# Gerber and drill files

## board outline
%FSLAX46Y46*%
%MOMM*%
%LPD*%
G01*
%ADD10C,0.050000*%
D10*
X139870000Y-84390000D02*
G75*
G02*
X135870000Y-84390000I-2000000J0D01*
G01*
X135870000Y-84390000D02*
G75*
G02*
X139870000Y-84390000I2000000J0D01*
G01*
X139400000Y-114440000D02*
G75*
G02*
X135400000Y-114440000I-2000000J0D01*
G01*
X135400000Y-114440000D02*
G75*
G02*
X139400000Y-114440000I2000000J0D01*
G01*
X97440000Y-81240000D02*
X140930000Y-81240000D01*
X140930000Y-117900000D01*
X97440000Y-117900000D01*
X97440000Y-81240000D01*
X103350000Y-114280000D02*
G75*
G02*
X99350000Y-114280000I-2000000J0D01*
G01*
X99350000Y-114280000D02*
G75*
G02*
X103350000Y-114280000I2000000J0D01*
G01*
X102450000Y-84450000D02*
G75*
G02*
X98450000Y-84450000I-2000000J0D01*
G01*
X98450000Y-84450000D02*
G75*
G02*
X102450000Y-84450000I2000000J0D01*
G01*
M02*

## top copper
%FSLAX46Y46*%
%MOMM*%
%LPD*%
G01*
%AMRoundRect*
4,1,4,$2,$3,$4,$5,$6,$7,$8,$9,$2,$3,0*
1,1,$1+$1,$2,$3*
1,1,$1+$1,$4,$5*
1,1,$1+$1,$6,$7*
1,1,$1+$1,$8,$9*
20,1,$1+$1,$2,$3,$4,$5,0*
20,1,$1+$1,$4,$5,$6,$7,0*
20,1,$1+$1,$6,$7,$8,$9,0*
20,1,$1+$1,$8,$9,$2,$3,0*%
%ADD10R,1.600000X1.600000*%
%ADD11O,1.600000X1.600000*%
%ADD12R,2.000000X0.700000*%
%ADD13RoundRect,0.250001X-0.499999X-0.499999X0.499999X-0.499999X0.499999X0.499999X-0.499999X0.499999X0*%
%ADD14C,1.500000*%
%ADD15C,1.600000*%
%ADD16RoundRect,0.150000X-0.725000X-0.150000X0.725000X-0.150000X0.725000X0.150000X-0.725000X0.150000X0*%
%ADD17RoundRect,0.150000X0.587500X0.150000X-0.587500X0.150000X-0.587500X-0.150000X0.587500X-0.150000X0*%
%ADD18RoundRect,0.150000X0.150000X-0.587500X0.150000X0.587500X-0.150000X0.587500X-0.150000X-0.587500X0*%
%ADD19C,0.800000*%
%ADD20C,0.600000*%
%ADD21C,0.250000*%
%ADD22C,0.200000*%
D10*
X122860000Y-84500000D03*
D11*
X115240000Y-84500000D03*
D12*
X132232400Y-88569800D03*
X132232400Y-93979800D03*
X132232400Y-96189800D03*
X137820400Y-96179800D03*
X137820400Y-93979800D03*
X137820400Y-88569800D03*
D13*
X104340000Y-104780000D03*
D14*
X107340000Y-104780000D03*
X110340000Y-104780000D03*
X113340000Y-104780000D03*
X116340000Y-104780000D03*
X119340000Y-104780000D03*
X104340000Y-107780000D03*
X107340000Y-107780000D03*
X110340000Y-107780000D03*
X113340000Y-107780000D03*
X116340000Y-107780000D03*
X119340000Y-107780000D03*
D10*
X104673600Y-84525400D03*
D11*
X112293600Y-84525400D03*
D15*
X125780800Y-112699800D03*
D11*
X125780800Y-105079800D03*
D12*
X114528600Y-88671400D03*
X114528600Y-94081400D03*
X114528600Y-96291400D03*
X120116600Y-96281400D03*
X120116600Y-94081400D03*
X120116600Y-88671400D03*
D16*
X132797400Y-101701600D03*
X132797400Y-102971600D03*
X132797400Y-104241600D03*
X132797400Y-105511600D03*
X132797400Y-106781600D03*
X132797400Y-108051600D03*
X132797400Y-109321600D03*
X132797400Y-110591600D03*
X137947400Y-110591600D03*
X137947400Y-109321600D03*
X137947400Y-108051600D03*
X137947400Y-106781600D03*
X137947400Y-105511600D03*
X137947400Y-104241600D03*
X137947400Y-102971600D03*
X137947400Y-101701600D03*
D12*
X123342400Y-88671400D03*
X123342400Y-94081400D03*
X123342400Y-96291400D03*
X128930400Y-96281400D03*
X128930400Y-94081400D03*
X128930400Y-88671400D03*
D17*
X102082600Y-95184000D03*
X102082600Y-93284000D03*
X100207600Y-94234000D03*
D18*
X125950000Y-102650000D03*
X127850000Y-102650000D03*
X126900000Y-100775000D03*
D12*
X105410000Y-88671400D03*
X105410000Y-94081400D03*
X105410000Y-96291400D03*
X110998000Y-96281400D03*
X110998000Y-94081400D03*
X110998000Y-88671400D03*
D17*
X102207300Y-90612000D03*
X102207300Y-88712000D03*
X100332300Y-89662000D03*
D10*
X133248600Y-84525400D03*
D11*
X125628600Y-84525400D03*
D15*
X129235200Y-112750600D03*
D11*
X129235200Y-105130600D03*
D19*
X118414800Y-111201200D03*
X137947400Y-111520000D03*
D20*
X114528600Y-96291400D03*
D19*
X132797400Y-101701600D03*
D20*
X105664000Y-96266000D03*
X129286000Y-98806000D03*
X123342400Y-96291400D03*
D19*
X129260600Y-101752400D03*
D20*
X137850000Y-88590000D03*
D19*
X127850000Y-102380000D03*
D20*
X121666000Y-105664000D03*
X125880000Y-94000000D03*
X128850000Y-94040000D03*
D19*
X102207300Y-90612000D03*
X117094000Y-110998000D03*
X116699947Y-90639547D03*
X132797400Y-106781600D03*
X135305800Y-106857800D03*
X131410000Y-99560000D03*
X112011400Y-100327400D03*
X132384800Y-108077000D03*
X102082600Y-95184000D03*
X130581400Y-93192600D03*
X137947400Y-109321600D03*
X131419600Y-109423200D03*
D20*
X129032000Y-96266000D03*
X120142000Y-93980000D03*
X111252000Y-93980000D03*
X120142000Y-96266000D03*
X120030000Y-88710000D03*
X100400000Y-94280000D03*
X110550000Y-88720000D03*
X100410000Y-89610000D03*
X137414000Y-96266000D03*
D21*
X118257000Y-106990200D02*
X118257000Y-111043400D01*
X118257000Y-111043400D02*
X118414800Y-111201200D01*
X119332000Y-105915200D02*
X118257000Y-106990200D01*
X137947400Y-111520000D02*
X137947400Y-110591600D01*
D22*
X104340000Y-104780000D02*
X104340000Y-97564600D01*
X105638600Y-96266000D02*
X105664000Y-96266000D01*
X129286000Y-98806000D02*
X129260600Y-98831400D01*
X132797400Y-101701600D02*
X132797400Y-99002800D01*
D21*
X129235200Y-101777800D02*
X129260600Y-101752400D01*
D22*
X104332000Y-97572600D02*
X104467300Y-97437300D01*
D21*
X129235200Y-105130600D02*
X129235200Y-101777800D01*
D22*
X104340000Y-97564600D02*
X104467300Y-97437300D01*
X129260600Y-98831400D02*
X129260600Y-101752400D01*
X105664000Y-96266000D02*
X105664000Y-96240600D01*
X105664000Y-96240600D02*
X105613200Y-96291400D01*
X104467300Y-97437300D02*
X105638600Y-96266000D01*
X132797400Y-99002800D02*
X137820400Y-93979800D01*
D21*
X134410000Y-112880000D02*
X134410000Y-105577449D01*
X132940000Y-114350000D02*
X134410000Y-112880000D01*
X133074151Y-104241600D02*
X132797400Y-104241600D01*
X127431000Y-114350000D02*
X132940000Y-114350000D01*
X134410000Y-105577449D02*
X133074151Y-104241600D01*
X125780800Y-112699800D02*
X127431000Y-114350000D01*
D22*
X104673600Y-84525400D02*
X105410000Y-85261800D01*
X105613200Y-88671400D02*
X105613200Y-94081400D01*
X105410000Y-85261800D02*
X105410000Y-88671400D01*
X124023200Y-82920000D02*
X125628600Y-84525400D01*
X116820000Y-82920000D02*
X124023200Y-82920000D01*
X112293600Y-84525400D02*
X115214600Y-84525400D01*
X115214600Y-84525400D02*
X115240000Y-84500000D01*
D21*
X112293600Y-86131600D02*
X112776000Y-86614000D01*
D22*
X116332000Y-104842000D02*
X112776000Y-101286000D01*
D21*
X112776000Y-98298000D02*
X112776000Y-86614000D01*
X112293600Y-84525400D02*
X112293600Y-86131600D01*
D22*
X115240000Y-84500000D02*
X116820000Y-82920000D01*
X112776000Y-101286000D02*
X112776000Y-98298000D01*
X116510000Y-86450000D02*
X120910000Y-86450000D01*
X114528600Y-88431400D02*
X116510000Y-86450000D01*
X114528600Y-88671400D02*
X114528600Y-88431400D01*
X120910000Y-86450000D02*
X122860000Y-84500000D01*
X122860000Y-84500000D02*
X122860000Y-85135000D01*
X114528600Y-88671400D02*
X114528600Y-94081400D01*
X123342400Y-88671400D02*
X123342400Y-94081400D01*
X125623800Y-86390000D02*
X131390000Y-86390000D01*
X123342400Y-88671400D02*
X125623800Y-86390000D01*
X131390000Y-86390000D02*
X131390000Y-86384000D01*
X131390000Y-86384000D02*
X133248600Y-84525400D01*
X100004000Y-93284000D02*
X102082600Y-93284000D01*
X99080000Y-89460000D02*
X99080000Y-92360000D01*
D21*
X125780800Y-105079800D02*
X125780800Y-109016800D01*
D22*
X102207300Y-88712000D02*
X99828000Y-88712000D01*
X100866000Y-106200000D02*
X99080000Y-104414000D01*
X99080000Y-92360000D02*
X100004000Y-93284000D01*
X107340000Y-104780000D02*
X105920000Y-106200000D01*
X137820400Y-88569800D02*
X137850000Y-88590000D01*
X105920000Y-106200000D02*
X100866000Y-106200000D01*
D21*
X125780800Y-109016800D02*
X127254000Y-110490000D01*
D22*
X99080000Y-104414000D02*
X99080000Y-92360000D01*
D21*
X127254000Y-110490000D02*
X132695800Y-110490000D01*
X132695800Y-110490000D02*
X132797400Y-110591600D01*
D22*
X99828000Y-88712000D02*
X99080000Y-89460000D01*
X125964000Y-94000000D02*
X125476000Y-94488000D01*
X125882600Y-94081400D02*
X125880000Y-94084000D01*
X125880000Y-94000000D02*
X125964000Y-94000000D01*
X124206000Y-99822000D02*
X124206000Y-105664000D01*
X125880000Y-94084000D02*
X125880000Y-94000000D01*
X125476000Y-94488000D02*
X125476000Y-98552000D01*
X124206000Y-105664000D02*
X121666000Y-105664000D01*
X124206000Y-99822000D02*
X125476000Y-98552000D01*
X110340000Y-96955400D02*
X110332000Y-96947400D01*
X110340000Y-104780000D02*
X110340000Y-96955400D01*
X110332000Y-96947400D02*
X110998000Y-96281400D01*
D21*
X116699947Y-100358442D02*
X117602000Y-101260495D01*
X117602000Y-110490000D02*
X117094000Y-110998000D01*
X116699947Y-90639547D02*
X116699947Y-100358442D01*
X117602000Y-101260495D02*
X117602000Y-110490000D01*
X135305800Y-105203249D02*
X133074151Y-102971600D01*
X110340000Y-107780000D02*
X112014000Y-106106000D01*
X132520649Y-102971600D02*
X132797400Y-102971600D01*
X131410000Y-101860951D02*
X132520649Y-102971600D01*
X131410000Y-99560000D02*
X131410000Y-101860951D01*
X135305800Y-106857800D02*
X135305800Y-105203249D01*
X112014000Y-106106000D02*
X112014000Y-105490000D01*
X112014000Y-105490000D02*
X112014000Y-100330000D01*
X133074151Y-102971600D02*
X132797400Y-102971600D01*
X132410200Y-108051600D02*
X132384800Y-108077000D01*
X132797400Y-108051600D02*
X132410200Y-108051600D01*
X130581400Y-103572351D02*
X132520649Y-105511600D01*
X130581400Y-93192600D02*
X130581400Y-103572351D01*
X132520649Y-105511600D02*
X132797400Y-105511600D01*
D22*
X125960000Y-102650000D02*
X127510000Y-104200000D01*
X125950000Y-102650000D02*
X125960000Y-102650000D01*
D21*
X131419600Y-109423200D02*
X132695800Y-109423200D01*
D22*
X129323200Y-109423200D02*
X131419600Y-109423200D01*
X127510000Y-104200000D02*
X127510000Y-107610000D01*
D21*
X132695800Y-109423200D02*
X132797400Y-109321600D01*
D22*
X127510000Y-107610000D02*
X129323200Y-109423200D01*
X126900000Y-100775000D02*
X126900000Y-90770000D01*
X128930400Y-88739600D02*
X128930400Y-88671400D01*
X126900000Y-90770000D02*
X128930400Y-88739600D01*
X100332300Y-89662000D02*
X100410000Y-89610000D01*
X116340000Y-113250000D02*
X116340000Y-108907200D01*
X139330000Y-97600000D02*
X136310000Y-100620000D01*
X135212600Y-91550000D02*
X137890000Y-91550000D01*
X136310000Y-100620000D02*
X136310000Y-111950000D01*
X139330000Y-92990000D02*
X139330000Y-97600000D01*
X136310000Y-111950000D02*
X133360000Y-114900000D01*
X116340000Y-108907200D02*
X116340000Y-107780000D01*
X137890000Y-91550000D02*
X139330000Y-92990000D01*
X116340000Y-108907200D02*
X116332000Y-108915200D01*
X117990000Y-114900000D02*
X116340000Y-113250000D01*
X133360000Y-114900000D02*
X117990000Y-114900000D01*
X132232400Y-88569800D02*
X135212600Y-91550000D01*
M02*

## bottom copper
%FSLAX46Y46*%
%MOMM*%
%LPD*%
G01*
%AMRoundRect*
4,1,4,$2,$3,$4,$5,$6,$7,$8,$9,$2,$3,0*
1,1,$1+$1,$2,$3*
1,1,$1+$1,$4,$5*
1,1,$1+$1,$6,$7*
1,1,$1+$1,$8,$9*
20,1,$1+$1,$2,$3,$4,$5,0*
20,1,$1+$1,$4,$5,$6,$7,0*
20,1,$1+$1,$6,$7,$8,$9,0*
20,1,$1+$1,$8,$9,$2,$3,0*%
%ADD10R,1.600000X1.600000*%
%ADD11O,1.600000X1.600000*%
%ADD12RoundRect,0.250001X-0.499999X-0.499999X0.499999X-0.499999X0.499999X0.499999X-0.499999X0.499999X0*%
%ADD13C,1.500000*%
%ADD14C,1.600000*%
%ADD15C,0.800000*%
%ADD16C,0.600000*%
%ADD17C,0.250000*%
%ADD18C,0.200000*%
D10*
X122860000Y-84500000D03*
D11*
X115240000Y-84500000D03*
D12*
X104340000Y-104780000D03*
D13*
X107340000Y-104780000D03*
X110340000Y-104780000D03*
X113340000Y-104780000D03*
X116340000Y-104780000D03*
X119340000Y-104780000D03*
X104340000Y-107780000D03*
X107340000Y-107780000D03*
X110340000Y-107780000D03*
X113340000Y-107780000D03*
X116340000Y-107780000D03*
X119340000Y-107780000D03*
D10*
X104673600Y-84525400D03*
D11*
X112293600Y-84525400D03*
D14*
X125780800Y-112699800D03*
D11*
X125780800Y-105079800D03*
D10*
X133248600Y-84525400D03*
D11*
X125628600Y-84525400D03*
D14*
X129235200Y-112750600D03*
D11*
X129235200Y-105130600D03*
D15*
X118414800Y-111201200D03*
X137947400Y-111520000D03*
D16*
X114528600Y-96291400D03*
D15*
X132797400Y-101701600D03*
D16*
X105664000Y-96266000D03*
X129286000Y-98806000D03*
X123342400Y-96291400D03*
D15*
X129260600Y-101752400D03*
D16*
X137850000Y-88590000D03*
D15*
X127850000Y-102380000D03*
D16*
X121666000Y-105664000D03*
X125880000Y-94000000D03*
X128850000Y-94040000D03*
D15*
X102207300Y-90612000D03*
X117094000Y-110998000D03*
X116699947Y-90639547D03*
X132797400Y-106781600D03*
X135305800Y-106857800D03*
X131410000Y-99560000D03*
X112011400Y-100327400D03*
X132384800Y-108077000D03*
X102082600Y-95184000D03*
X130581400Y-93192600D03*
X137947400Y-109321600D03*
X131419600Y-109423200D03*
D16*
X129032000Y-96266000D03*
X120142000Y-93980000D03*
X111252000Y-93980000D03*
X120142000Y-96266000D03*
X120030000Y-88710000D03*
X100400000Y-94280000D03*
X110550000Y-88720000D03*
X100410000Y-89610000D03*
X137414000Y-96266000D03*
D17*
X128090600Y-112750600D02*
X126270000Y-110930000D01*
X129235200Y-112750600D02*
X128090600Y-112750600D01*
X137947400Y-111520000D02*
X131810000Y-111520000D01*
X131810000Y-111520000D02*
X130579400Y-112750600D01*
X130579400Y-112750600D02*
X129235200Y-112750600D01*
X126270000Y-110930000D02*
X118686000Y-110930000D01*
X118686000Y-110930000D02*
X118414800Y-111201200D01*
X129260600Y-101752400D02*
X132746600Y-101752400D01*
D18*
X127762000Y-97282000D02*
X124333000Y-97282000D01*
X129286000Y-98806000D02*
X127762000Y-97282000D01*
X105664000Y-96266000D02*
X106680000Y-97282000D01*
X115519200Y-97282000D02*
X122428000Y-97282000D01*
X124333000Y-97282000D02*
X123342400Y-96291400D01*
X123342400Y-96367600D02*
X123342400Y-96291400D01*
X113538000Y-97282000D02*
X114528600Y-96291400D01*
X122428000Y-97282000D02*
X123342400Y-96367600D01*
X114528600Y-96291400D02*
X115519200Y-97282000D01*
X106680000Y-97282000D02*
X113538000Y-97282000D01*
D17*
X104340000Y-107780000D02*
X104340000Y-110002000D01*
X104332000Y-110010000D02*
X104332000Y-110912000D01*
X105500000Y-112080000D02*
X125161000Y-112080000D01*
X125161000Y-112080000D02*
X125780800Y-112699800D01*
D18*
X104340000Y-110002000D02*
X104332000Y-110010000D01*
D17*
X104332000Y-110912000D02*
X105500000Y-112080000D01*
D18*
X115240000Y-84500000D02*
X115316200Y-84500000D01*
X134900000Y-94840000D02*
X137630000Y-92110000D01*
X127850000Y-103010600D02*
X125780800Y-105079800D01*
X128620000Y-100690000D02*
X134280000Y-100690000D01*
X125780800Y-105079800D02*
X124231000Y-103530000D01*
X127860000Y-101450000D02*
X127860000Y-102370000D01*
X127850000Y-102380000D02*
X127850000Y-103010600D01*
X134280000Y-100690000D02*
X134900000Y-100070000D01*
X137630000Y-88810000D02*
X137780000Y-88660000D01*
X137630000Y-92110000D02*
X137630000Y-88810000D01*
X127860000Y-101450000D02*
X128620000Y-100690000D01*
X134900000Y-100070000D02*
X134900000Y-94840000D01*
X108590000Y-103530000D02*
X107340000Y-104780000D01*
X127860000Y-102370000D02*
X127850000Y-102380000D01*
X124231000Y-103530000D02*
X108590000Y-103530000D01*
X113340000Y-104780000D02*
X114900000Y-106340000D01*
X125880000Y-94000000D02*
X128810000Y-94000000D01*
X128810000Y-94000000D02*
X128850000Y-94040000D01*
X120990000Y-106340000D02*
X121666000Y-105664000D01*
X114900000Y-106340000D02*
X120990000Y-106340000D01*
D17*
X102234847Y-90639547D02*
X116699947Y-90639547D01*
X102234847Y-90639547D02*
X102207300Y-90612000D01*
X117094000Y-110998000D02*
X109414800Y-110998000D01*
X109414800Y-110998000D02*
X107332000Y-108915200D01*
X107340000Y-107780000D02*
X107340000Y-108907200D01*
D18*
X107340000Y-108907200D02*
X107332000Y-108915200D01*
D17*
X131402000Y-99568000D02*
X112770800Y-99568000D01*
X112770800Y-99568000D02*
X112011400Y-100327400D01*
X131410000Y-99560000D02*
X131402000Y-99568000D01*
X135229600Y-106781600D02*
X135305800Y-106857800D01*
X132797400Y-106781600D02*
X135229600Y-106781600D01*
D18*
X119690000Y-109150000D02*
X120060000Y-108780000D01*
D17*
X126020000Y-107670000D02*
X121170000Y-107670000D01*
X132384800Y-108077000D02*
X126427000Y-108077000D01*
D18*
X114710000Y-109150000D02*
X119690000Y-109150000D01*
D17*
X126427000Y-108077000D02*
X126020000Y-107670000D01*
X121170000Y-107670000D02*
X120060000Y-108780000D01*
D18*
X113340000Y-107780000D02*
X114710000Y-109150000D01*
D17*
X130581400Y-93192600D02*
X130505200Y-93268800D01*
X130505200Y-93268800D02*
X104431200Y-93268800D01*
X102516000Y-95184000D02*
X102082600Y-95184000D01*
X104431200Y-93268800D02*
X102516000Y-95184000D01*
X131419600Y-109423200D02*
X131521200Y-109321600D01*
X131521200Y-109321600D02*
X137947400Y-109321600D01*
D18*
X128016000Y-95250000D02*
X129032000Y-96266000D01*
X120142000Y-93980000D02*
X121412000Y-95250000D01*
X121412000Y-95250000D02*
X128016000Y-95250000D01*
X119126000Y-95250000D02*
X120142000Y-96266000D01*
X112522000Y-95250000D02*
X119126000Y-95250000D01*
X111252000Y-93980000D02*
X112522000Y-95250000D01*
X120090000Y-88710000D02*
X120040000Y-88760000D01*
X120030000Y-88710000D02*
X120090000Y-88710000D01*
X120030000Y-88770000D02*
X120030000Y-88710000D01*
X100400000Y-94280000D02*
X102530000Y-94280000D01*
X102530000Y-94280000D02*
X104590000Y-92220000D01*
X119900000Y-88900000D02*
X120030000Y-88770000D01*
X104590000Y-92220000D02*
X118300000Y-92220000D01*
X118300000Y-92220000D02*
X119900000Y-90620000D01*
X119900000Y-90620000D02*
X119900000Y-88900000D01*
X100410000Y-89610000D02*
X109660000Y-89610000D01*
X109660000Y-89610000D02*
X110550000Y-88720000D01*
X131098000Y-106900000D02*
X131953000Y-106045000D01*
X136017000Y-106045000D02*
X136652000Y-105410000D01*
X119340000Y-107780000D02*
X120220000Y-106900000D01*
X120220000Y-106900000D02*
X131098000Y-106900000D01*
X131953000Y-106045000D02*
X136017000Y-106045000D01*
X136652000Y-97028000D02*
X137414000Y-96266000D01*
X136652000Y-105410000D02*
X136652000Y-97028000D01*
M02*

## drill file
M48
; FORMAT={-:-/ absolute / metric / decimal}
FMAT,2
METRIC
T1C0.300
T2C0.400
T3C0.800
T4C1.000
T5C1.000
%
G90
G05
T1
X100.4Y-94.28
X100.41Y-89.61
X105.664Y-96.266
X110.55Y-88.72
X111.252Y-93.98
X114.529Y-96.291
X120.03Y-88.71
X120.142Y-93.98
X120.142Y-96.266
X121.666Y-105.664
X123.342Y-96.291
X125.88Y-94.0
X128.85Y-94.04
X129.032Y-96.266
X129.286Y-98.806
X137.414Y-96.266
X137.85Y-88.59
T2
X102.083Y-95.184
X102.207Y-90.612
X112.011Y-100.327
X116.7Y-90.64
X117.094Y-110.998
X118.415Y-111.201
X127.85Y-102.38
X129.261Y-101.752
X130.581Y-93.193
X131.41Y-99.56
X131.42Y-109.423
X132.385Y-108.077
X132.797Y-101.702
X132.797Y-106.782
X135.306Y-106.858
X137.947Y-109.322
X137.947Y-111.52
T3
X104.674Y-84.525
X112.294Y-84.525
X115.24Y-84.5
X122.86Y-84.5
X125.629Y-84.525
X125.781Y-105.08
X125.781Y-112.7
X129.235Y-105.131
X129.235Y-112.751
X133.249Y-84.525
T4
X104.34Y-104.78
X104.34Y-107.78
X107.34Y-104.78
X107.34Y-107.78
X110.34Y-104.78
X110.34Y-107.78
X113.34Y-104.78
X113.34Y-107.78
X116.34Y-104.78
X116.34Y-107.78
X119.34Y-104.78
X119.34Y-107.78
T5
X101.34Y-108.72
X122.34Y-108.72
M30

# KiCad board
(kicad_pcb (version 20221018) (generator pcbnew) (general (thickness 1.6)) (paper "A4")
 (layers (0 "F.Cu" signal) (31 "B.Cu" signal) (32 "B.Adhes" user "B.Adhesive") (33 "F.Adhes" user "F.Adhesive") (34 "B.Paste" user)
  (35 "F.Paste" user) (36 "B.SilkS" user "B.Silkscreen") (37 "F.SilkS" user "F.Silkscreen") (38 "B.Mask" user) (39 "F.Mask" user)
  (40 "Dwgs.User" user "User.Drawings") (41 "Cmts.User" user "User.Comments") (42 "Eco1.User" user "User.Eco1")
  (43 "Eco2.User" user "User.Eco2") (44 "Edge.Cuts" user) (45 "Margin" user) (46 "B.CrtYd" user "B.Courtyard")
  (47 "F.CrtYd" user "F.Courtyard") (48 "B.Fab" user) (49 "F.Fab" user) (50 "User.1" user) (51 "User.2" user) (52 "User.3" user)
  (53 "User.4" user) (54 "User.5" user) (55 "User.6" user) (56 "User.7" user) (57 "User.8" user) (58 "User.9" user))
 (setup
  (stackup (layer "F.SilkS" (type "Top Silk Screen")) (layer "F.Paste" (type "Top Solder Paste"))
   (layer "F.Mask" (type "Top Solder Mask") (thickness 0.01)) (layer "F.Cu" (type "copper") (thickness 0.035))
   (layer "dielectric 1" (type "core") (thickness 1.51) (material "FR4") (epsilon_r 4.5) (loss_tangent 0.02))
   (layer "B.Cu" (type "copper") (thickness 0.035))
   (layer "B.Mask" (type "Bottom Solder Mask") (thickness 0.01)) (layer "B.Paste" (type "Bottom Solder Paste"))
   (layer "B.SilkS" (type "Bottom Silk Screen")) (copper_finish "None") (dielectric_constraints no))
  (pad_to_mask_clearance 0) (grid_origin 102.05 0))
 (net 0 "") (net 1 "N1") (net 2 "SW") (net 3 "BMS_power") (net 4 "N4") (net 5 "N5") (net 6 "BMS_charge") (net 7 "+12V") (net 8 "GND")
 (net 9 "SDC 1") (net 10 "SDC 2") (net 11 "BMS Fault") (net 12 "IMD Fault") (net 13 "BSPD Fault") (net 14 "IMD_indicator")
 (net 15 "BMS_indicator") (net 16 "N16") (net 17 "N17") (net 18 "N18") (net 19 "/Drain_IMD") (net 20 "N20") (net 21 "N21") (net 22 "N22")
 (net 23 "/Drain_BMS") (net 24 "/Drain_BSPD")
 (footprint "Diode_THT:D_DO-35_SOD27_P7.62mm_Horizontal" (layer "F.Cu") (at 122.86 84.5 180)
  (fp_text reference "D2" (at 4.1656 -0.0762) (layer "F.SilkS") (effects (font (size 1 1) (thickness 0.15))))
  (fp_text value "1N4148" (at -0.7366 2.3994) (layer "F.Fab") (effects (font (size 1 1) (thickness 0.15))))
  (pad "1" thru_hole rect (at 0 0 180) (size 1.6 1.6) (drill 0.8) (layers "*.Cu" "*.Mask") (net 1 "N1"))
  (pad "2" thru_hole oval (at 7.62 0 180) (size 1.6 1.6) (drill 0.8) (layers "*.Cu" "*.Mask") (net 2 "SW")))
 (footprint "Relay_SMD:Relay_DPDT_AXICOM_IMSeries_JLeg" (layer "F.Cu") (at 135.0264 92.3798)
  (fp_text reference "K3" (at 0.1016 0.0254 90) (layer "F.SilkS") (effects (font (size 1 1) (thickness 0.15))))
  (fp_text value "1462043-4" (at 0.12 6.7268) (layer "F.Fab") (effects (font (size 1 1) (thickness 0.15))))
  (pad "1" smd rect (at -2.794 -3.81) (size 2 0.7) (layers "F.Cu" "F.Paste" "F.Mask") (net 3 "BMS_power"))
  (pad "3" smd rect (at -2.794 1.6) (size 2 0.7) (layers "F.Cu" "F.Paste" "F.Mask") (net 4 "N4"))
  (pad "4" smd rect (at -2.794 3.81) (size 2 0.7) (layers "F.Cu" "F.Paste" "F.Mask") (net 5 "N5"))
  (pad "5" smd rect (at 2.794 3.8) (size 2 0.7) (layers "F.Cu" "F.Paste" "F.Mask") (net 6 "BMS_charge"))
  (pad "6" smd rect (at 2.794 1.6) (size 2 0.7) (layers "F.Cu" "F.Paste" "F.Mask") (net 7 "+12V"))
  (pad "8" smd rect (at 2.794 -3.81) (size 2 0.7) (layers "F.Cu" "F.Paste" "F.Mask") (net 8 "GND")))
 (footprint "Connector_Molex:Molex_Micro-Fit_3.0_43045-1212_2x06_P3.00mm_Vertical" (layer "F.Cu") (at 104.34 104.78)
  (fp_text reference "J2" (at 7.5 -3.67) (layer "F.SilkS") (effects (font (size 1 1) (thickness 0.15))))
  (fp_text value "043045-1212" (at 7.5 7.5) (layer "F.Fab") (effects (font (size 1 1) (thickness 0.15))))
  (pad "" np_thru_hole circle (at -3 3.94) (size 1 1) (drill 1) (layers "*.Cu" "*.Mask"))
  (pad "" np_thru_hole circle (at 18 3.94) (size 1 1) (drill 1) (layers "*.Cu" "*.Mask"))
  (pad "1" thru_hole roundrect (at 0 0) (size 1.5 1.5) (drill 1) (layers "*.Cu" "*.Mask") (roundrect_rratio 0.1666673333) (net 7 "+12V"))
  (pad "2" thru_hole circle (at 3 0) (size 1.5 1.5) (drill 1) (layers "*.Cu" "*.Mask") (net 8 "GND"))
  (pad "3" thru_hole circle (at 6 0) (size 1.5 1.5) (drill 1) (layers "*.Cu" "*.Mask") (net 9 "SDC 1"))
  (pad "4" thru_hole circle (at 9 0) (size 1.5 1.5) (drill 1) (layers "*.Cu" "*.Mask") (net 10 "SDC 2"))
  (pad "5" thru_hole circle (at 12 0) (size 1.5 1.5) (drill 1) (layers "*.Cu" "*.Mask") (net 2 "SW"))
  (pad "6" thru_hole circle (at 15 0) (size 1.5 1.5) (drill 1) (layers "*.Cu" "*.Mask") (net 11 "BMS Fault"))
  (pad "7" thru_hole circle (at 0 3) (size 1.5 1.5) (drill 1) (layers "*.Cu" "*.Mask") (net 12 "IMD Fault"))
  (pad "8" thru_hole circle (at 3 3) (size 1.5 1.5) (drill 1) (layers "*.Cu" "*.Mask") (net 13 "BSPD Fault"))
  (pad "9" thru_hole circle (at 6 3) (size 1.5 1.5) (drill 1) (layers "*.Cu" "*.Mask") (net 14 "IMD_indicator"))
  (pad "10" thru_hole circle (at 9 3) (size 1.5 1.5) (drill 1) (layers "*.Cu" "*.Mask") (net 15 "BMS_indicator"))
  (pad "11" thru_hole circle (at 12 3) (size 1.5 1.5) (drill 1) (layers "*.Cu" "*.Mask") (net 3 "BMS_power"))
  (pad "12" thru_hole circle (at 15 3) (size 1.5 1.5) (drill 1) (layers "*.Cu" "*.Mask") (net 6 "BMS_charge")))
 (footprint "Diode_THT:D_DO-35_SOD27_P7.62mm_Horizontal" (layer "F.Cu") (at 104.6736 84.5254)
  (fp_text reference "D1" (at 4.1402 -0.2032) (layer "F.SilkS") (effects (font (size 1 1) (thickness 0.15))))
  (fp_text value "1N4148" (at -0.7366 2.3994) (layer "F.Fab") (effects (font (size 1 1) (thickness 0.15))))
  (pad "1" thru_hole rect (at 0 0) (size 1.6 1.6) (drill 0.8) (layers "*.Cu" "*.Mask") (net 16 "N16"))
  (pad "2" thru_hole oval (at 7.62 0) (size 1.6 1.6) (drill 0.8) (layers "*.Cu" "*.Mask") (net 2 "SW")))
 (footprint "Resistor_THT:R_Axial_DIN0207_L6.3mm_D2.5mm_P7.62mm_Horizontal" (layer "F.Cu") (at 125.7808 112.6998 90)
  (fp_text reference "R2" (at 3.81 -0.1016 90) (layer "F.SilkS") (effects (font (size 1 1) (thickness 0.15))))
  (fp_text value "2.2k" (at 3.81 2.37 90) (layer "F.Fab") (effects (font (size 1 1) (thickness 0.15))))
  (pad "1" thru_hole circle (at 0 0 90) (size 1.6 1.6) (drill 0.8) (layers "*.Cu" "*.Mask") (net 12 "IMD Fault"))
  (pad "2" thru_hole oval (at 7.62 0 90) (size 1.6 1.6) (drill 0.8) (layers "*.Cu" "*.Mask") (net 8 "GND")))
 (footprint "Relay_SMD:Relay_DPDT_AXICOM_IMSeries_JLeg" (layer "F.Cu") (at 117.3226 92.4814)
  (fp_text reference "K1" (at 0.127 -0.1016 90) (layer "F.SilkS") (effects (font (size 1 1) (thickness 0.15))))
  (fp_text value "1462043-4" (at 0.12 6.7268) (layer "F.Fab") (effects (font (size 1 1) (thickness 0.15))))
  (pad "1" smd rect (at -2.794 -3.81) (size 2 0.7) (layers "F.Cu" "F.Paste" "F.Mask") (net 1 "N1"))
  (pad "3" smd rect (at -2.794 1.6) (size 2 0.7) (layers "F.Cu" "F.Paste" "F.Mask") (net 1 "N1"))
  (pad "4" smd rect (at -2.794 3.81) (size 2 0.7) (layers "F.Cu" "F.Paste" "F.Mask") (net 7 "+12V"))
  (pad "5" smd rect (at 2.794 3.8) (size 2 0.7) (layers "F.Cu" "F.Paste" "F.Mask") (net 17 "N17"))
  (pad "6" smd rect (at 2.794 1.6) (size 2 0.7) (layers "F.Cu" "F.Paste" "F.Mask") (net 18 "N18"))
  (pad "8" smd rect (at 2.794 -3.81) (size 2 0.7) (layers "F.Cu" "F.Paste" "F.Mask") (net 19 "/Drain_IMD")))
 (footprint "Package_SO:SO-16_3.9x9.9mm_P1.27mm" (layer "F.Cu") (at 135.3724 106.1466)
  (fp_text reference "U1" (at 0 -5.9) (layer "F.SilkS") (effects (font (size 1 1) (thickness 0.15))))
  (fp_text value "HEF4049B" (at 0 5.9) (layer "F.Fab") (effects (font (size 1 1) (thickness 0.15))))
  (pad "1" smd roundrect (at -2.575 -4.445) (size 1.75 0.6) (layers "F.Cu" "F.Paste" "F.Mask") (roundrect_rratio 0.25) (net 7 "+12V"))
  (pad "2" smd roundrect (at -2.575 -3.175) (size 1.75 0.6) (layers "F.Cu" "F.Paste" "F.Mask") (roundrect_rratio 0.25)
   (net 14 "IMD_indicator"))
  (pad "3" smd roundrect (at -2.575 -1.905) (size 1.75 0.6) (layers "F.Cu" "F.Paste" "F.Mask") (roundrect_rratio 0.25) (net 12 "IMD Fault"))
  (pad "4" smd roundrect (at -2.575 -0.635) (size 1.75 0.6) (layers "F.Cu" "F.Paste" "F.Mask") (roundrect_rratio 0.25) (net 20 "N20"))
  (pad "5" smd roundrect (at -2.575 0.635) (size 1.75 0.6) (layers "F.Cu" "F.Paste" "F.Mask") (roundrect_rratio 0.25)
   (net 14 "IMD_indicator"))
  (pad "6" smd roundrect (at -2.575 1.905) (size 1.75 0.6) (layers "F.Cu" "F.Paste" "F.Mask") (roundrect_rratio 0.25)
   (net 15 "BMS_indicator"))
  (pad "7" smd roundrect (at -2.575 3.175) (size 1.75 0.6) (layers "F.Cu" "F.Paste" "F.Mask") (roundrect_rratio 0.25) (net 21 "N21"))
  (pad "8" smd roundrect (at -2.575 4.445) (size 1.75 0.6) (layers "F.Cu" "F.Paste" "F.Mask") (roundrect_rratio 0.25) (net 8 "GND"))
  (pad "9" smd roundrect (at 2.575 4.445) (size 1.75 0.6) (layers "F.Cu" "F.Paste" "F.Mask") (roundrect_rratio 0.25) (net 11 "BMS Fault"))
  (pad "10" smd roundrect (at 2.575 3.175) (size 1.75 0.6) (layers "F.Cu" "F.Paste" "F.Mask") (roundrect_rratio 0.25) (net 21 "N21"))
  (pad "11" smd roundrect (at 2.575 1.905) (size 1.75 0.6) (layers "F.Cu" "F.Paste" "F.Mask") (roundrect_rratio 0.25))
  (pad "12" smd roundrect (at 2.575 0.635) (size 1.75 0.6) (layers "F.Cu" "F.Paste" "F.Mask") (roundrect_rratio 0.25))
  (pad "13" smd roundrect (at 2.575 -0.635) (size 1.75 0.6) (layers "F.Cu" "F.Paste" "F.Mask") (roundrect_rratio 0.25))
  (pad "14" smd roundrect (at 2.575 -1.905) (size 1.75 0.6) (layers "F.Cu" "F.Paste" "F.Mask") (roundrect_rratio 0.25))
  (pad "15" smd roundrect (at 2.575 -3.175) (size 1.75 0.6) (layers "F.Cu" "F.Paste" "F.Mask") (roundrect_rratio 0.25))
  (pad "16" smd roundrect (at 2.575 -4.445) (size 1.75 0.6) (layers "F.Cu" "F.Paste" "F.Mask") (roundrect_rratio 0.25)))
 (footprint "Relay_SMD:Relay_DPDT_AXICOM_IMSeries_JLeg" (layer "F.Cu") (at 126.1364 92.4814)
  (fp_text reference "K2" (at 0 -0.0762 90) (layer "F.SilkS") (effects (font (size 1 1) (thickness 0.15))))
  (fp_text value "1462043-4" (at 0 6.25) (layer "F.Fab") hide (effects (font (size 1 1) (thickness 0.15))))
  (pad "1" smd rect (at -2.794 -3.81) (size 2 0.7) (layers "F.Cu" "F.Paste" "F.Mask") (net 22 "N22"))
  (pad "3" smd rect (at -2.794 1.6) (size 2 0.7) (layers "F.Cu" "F.Paste" "F.Mask") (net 22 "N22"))
  (pad "4" smd rect (at -2.794 3.81) (size 2 0.7) (layers "F.Cu" "F.Paste" "F.Mask") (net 7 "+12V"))
  (pad "5" smd rect (at 2.794 3.8) (size 2 0.7) (layers "F.Cu" "F.Paste" "F.Mask") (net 18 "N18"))
  (pad "6" smd rect (at 2.794 1.6) (size 2 0.7) (layers "F.Cu" "F.Paste" "F.Mask") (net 10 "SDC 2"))
  (pad "8" smd rect (at 2.794 -3.81) (size 2 0.7) (layers "F.Cu" "F.Paste" "F.Mask") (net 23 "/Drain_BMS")))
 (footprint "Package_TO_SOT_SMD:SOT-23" (layer "F.Cu") (at 101.1451 94.234 180)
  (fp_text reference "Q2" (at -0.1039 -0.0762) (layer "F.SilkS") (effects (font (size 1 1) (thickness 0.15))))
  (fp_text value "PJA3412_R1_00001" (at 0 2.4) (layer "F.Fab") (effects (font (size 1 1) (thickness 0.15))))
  (pad "1" smd roundrect (at -0.9375 -0.95 180) (size 1.475 0.6) (layers "F.Cu" "F.Paste" "F.Mask") (roundrect_rratio 0.25) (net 20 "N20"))
  (pad "2" smd roundrect (at -0.9375 0.95 180) (size 1.475 0.6) (layers "F.Cu" "F.Paste" "F.Mask") (roundrect_rratio 0.25) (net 8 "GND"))
  (pad "3" smd roundrect (at 0.9375 0 180) (size 1.475 0.6) (layers "F.Cu" "F.Paste" "F.Mask") (roundrect_rratio 0.25) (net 19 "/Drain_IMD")))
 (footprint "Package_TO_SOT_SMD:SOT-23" (layer "F.Cu") (at 126.9 101.7125 90)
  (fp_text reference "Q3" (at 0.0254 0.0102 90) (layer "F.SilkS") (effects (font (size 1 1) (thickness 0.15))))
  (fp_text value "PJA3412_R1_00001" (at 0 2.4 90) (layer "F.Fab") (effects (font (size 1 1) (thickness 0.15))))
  (pad "1" smd roundrect (at -0.9375 -0.95 90) (size 1.475 0.6) (layers "F.Cu" "F.Paste" "F.Mask") (roundrect_rratio 0.25) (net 21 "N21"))
  (pad "2" smd roundrect (at -0.9375 0.95 90) (size 1.475 0.6) (layers "F.Cu" "F.Paste" "F.Mask") (roundrect_rratio 0.25) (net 8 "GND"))
  (pad "3" smd roundrect (at 0.9375 0 90) (size 1.475 0.6) (layers "F.Cu" "F.Paste" "F.Mask") (roundrect_rratio 0.25) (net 23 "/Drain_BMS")))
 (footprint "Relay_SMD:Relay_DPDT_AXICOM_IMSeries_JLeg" (layer "F.Cu") (at 108.204 92.4814)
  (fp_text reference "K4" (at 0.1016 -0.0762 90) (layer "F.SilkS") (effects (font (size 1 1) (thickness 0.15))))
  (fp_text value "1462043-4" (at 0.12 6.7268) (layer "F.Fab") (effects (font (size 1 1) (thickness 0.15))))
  (pad "1" smd rect (at -2.794 -3.81) (size 2 0.7) (layers "F.Cu" "F.Paste" "F.Mask") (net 16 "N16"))
  (pad "3" smd rect (at -2.794 1.6) (size 2 0.7) (layers "F.Cu" "F.Paste" "F.Mask") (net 16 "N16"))
  (pad "4" smd rect (at -2.794 3.81) (size 2 0.7) (layers "F.Cu" "F.Paste" "F.Mask") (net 7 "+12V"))
  (pad "5" smd rect (at 2.794 3.8) (size 2 0.7) (layers "F.Cu" "F.Paste" "F.Mask") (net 9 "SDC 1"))
  (pad "6" smd rect (at 2.794 1.6) (size 2 0.7) (layers "F.Cu" "F.Paste" "F.Mask") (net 17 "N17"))
  (pad "8" smd rect (at 2.794 -3.81) (size 2 0.7) (layers "F.Cu" "F.Paste" "F.Mask") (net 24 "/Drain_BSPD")))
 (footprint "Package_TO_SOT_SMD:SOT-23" (layer "F.Cu") (at 101.2698 89.662 180)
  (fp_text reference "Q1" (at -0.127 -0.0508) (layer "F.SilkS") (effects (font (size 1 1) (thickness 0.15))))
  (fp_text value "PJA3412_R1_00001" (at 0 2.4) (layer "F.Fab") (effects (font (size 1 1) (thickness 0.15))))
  (pad "1" smd roundrect (at -0.9375 -0.95 180) (size 1.475 0.6) (layers "F.Cu" "F.Paste" "F.Mask") (roundrect_rratio 0.25)
   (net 13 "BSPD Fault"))
  (pad "2" smd roundrect (at -0.9375 0.95 180) (size 1.475 0.6) (layers "F.Cu" "F.Paste" "F.Mask") (roundrect_rratio 0.25) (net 8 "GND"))
  (pad "3" smd roundrect (at 0.9375 0 180) (size 1.475 0.6) (layers "F.Cu" "F.Paste" "F.Mask") (roundrect_rratio 0.25)
   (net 24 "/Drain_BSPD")))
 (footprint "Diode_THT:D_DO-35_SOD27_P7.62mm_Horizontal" (layer "F.Cu") (at 133.2486 84.5254 180)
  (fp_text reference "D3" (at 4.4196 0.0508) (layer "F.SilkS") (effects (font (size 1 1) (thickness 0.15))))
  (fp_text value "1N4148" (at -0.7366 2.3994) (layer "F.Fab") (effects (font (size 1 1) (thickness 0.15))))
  (pad "1" thru_hole rect (at 0 0 180) (size 1.6 1.6) (drill 0.8) (layers "*.Cu" "*.Mask") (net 22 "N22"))
  (pad "2" thru_hole oval (at 7.62 0 180) (size 1.6 1.6) (drill 0.8) (layers "*.Cu" "*.Mask") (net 2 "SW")))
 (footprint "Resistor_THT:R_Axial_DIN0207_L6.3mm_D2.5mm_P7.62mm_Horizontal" (layer "F.Cu") (at 129.2352 112.7506 90)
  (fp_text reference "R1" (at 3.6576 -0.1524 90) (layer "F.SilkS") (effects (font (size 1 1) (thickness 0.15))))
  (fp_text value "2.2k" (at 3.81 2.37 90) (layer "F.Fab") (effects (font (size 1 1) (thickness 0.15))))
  (pad "1" thru_hole circle (at 0 0 90) (size 1.6 1.6) (drill 0.8) (layers "*.Cu" "*.Mask") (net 11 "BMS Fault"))
  (pad "2" thru_hole oval (at 7.62 0 90) (size 1.6 1.6) (drill 0.8) (layers "*.Cu" "*.Mask") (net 7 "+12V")))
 (gr_circle (center 137.87 84.39) (end 139.87 84.39) (stroke (width 0.05) (type default)) (fill none) (layer "Edge.Cuts"))
 (gr_circle (center 137.4 114.44) (end 139.4 114.44) (stroke (width 0.05) (type default)) (fill none) (layer "Edge.Cuts"))
 (gr_rect (start 97.44 81.24) (end 140.93 117.9) (stroke (width 0.05) (type default)) (fill none) (layer "Edge.Cuts"))
 (gr_circle (center 101.35 114.28) (end 103.35 114.28) (stroke (width 0.05) (type default)) (fill none) (layer "Edge.Cuts"))
 (gr_circle (center 100.45 84.45) (end 102.45 84.45) (stroke (width 0.05) (type default)) (fill none) (layer "Edge.Cuts"))
 (segment (start 118.257 106.9902) (end 118.257 111.0434) (width 0.25) (layer "F.Cu") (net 11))
 (segment (start 118.257 111.0434) (end 118.4148 111.2012) (width 0.25) (layer "F.Cu") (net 11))
 (segment (start 119.332 105.9152) (end 118.257 106.9902) (width 0.25) (layer "F.Cu") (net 11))
 (segment (start 137.9474 111.52) (end 137.9474 110.5916) (width 0.25) (layer "F.Cu") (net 11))
 (via (at 118.4148 111.2012) (size 0.8) (drill 0.4) (layers "F.Cu" "B.Cu") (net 11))
 (via (at 137.9474 111.52) (size 0.8) (drill 0.4) (layers "F.Cu" "B.Cu") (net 11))
 (segment (start 128.0906 112.7506) (end 126.27 110.93) (width 0.25) (layer "B.Cu") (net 11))
 (segment (start 129.2352 112.7506) (end 128.0906 112.7506) (width 0.25) (layer "B.Cu") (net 11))
 (segment (start 137.9474 111.52) (end 131.81 111.52) (width 0.25) (layer "B.Cu") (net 11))
 (segment (start 131.81 111.52) (end 130.5794 112.7506) (width 0.25) (layer "B.Cu") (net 11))
 (segment (start 130.5794 112.7506) (end 129.2352 112.7506) (width 0.25) (layer "B.Cu") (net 11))
 (segment (start 126.27 110.93) (end 118.686 110.93) (width 0.25) (layer "B.Cu") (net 11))
 (segment (start 118.686 110.93) (end 118.4148 111.2012) (width 0.25) (layer "B.Cu") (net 11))
 (segment (start 104.34 104.78) (end 104.34 97.5646) (width 0.2) (layer "F.Cu") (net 7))
 (segment (start 105.6386 96.266) (end 105.664 96.266) (width 0.2) (layer "F.Cu") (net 7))
 (segment (start 129.286 98.806) (end 129.2606 98.8314) (width 0.2) (layer "F.Cu") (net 7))
 (segment (start 132.7974 101.7016) (end 132.7974 99.0028) (width 0.2) (layer "F.Cu") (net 7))
 (segment (start 129.2352 101.7778) (end 129.2606 101.7524) (width 0.25) (layer "F.Cu") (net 7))
 (segment (start 104.332 97.5726) (end 104.4673 97.4373) (width 0.2) (layer "F.Cu") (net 7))
 (segment (start 129.2352 105.1306) (end 129.2352 101.7778) (width 0.25) (layer "F.Cu") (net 7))
 (segment (start 104.34 97.5646) (end 104.4673 97.4373) (width 0.2) (layer "F.Cu") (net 7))
 (segment (start 129.2606 98.8314) (end 129.2606 101.7524) (width 0.2) (layer "F.Cu") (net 7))
 (segment (start 105.664 96.266) (end 105.664 96.2406) (width 0.2) (layer "F.Cu") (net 7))
 (segment (start 105.664 96.2406) (end 105.6132 96.2914) (width 0.2) (layer "F.Cu") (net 7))
 (segment (start 104.4673 97.4373) (end 105.6386 96.266) (width 0.2) (layer "F.Cu") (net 7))
 (segment (start 132.7974 99.0028) (end 137.8204 93.9798) (width 0.2) (layer "F.Cu") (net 7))
 (via (at 114.5286 96.2914) (size 0.6) (drill 0.3) (layers "F.Cu" "B.Cu") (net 7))
 (via (at 132.7974 101.7016) (size 0.8) (drill 0.4) (layers "F.Cu" "B.Cu") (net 7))
 (via (at 105.664 96.266) (size 0.6) (drill 0.3) (layers "F.Cu" "B.Cu") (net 7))
 (via (at 129.286 98.806) (size 0.6) (drill 0.3) (layers "F.Cu" "B.Cu") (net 7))
 (via (at 123.3424 96.2914) (size 0.6) (drill 0.3) (layers "F.Cu" "B.Cu") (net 7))
 (via (at 129.2606 101.7524) (size 0.8) (drill 0.4) (layers "F.Cu" "B.Cu") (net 7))
 (segment (start 129.2606 101.7524) (end 132.7466 101.7524) (width 0.25) (layer "B.Cu") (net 7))
 (segment (start 127.762 97.282) (end 124.333 97.282) (width 0.2) (layer "B.Cu") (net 7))
 (segment (start 129.286 98.806) (end 127.762 97.282) (width 0.2) (layer "B.Cu") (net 7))
 (segment (start 105.664 96.266) (end 106.68 97.282) (width 0.2) (layer "B.Cu") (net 7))
 (segment (start 115.5192 97.282) (end 122.428 97.282) (width 0.2) (layer "B.Cu") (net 7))
 (segment (start 124.333 97.282) (end 123.3424 96.2914) (width 0.2) (layer "B.Cu") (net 7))
 (segment (start 123.3424 96.3676) (end 123.3424 96.2914) (width 0.2) (layer "B.Cu") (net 7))
 (segment (start 113.538 97.282) (end 114.5286 96.2914) (width 0.2) (layer "B.Cu") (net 7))
 (segment (start 122.428 97.282) (end 123.3424 96.3676) (width 0.2) (layer "B.Cu") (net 7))
 (segment (start 114.5286 96.2914) (end 115.5192 97.282) (width 0.2) (layer "B.Cu") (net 7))
 (segment (start 106.68 97.282) (end 113.538 97.282) (width 0.2) (layer "B.Cu") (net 7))
 (segment (start 134.41 112.88) (end 134.41 105.577449) (width 0.25) (layer "F.Cu") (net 12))
 (segment (start 132.94 114.35) (end 134.41 112.88) (width 0.25) (layer "F.Cu") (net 12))
 (segment (start 133.074151 104.2416) (end 132.7974 104.2416) (width 0.25) (layer "F.Cu") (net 12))
 (segment (start 127.431 114.35) (end 132.94 114.35) (width 0.25) (layer "F.Cu") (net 12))
 (segment (start 134.41 105.577449) (end 133.074151 104.2416) (width 0.25) (layer "F.Cu") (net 12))
 (segment (start 125.7808 112.6998) (end 127.431 114.35) (width 0.25) (layer "F.Cu") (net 12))
 (segment (start 104.34 107.78) (end 104.34 110.002) (width 0.25) (layer "B.Cu") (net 12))
 (segment (start 104.332 110.01) (end 104.332 110.912) (width 0.25) (layer "B.Cu") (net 12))
 (segment (start 105.5 112.08) (end 125.161 112.08) (width 0.25) (layer "B.Cu") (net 12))
 (segment (start 125.161 112.08) (end 125.7808 112.6998) (width 0.25) (layer "B.Cu") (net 12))
 (segment (start 104.34 110.002) (end 104.332 110.01) (width 0.2) (layer "B.Cu") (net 12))
 (segment (start 104.332 110.912) (end 105.5 112.08) (width 0.25) (layer "B.Cu") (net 12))
 (segment (start 104.6736 84.5254) (end 105.41 85.2618) (width 0.2) (layer "F.Cu") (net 16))
 (segment (start 105.6132 88.6714) (end 105.6132 94.0814) (width 0.2) (layer "F.Cu") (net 16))
 (segment (start 105.41 85.2618) (end 105.41 88.6714) (width 0.2) (layer "F.Cu") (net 16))
 (segment (start 124.0232 82.92) (end 125.6286 84.5254) (width 0.2) (layer "F.Cu") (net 2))
 (segment (start 116.82 82.92) (end 124.0232 82.92) (width 0.2) (layer "F.Cu") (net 2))
 (segment (start 112.2936 84.5254) (end 115.2146 84.5254) (width 0.2) (layer "F.Cu") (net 2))
 (segment (start 115.2146 84.5254) (end 115.24 84.5) (width 0.2) (layer "F.Cu") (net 2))
 (segment (start 112.2936 86.1316) (end 112.776 86.614) (width 0.25) (layer "F.Cu") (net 2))
 (segment (start 116.332 104.842) (end 112.776 101.286) (width 0.2) (layer "F.Cu") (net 2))
 (segment (start 112.776 98.298) (end 112.776 86.614) (width 0.25) (layer "F.Cu") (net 2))
 (segment (start 112.2936 84.5254) (end 112.2936 86.1316) (width 0.25) (layer "F.Cu") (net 2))
 (segment (start 115.24 84.5) (end 116.82 82.92) (width 0.2) (layer "F.Cu") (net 2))
 (segment (start 112.776 101.286) (end 112.776 98.298) (width 0.2) (layer "F.Cu") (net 2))
 (segment (start 115.24 84.5) (end 115.3162 84.5) (width 0.2) (layer "B.Cu") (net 2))
 (segment (start 116.51 86.45) (end 120.91 86.45) (width 0.2) (layer "F.Cu") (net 1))
 (segment (start 114.5286 88.4314) (end 116.51 86.45) (width 0.2) (layer "F.Cu") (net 1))
 (segment (start 114.5286 88.6714) (end 114.5286 88.4314) (width 0.2) (layer "F.Cu") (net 1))
 (segment (start 120.91 86.45) (end 122.86 84.5) (width 0.2) (layer "F.Cu") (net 1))
 (segment (start 122.86 84.5) (end 122.86 85.135) (width 0.2) (layer "F.Cu") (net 1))
 (segment (start 114.5286 88.6714) (end 114.5286 94.0814) (width 0.2) (layer "F.Cu") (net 1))
 (segment (start 123.3424 88.6714) (end 123.3424 94.0814) (width 0.2) (layer "F.Cu") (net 22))
 (segment (start 125.6238 86.39) (end 131.39 86.39) (width 0.2) (layer "F.Cu") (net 22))
 (segment (start 123.3424 88.6714) (end 125.6238 86.39) (width 0.2) (layer "F.Cu") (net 22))
 (segment (start 131.39 86.39) (end 131.39 86.384) (width 0.2) (layer "F.Cu") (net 22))
 (segment (start 131.39 86.384) (end 133.2486 84.5254) (width 0.2) (layer "F.Cu") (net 22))
 (segment (start 100.004 93.284) (end 102.0826 93.284) (width 0.2) (layer "F.Cu") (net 8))
 (segment (start 99.08 89.46) (end 99.08 92.36) (width 0.2) (layer "F.Cu") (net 8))
 (segment (start 125.7808 105.0798) (end 125.7808 109.0168) (width 0.25) (layer "F.Cu") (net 8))
 (segment (start 102.2073 88.712) (end 99.828 88.712) (width 0.2) (layer "F.Cu") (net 8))
 (segment (start 100.866 106.2) (end 99.08 104.414) (width 0.2) (layer "F.Cu") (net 8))
 (segment (start 99.08 92.36) (end 100.004 93.284) (width 0.2) (layer "F.Cu") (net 8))
 (segment (start 107.34 104.78) (end 105.92 106.2) (width 0.2) (layer "F.Cu") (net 8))
 (segment (start 137.8204 88.5698) (end 137.85 88.59) (width 0.2) (layer "F.Cu") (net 8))
 (segment (start 105.92 106.2) (end 100.866 106.2) (width 0.2) (layer "F.Cu") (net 8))
 (segment (start 125.7808 109.0168) (end 127.254 110.49) (width 0.25) (layer "F.Cu") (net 8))
 (segment (start 99.08 104.414) (end 99.08 92.36) (width 0.2) (layer "F.Cu") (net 8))
 (segment (start 127.254 110.49) (end 132.6958 110.49) (width 0.25) (layer "F.Cu") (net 8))
 (segment (start 132.6958 110.49) (end 132.7974 110.5916) (width 0.25) (layer "F.Cu") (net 8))
 (segment (start 99.828 88.712) (end 99.08 89.46) (width 0.2) (layer "F.Cu") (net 8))
 (via (at 137.85 88.59) (size 0.6) (drill 0.3) (layers "F.Cu" "B.Cu") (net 8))
 (via (at 127.85 102.38) (size 0.8) (drill 0.4) (layers "F.Cu" "B.Cu") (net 8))
 (segment (start 134.9 94.84) (end 137.63 92.11) (width 0.2) (layer "B.Cu") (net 8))
 (segment (start 127.85 103.0106) (end 125.7808 105.0798) (width 0.2) (layer "B.Cu") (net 8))
 (segment (start 128.62 100.69) (end 134.28 100.69) (width 0.2) (layer "B.Cu") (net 8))
 (segment (start 125.7808 105.0798) (end 124.231 103.53) (width 0.2) (layer "B.Cu") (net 8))
 (segment (start 127.86 101.45) (end 127.86 102.37) (width 0.2) (layer "B.Cu") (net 8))
 (segment (start 127.85 102.38) (end 127.85 103.0106) (width 0.2) (layer "B.Cu") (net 8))
 (segment (start 134.28 100.69) (end 134.9 100.07) (width 0.2) (layer "B.Cu") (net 8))
 (segment (start 137.63 88.81) (end 137.78 88.66) (width 0.2) (layer "B.Cu") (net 8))
 (segment (start 137.63 92.11) (end 137.63 88.81) (width 0.2) (layer "B.Cu") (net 8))
 (segment (start 127.86 101.45) (end 128.62 100.69) (width 0.2) (layer "B.Cu") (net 8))
 (segment (start 134.9 100.07) (end 134.9 94.84) (width 0.2) (layer "B.Cu") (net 8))
 (segment (start 108.59 103.53) (end 107.34 104.78) (width 0.2) (layer "B.Cu") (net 8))
 (segment (start 127.86 102.37) (end 127.85 102.38) (width 0.2) (layer "B.Cu") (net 8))
 (segment (start 124.231 103.53) (end 108.59 103.53) (width 0.2) (layer "B.Cu") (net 8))
 (segment (start 125.964 94) (end 125.476 94.488) (width 0.2) (layer "F.Cu") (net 10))
 (segment (start 125.8826 94.0814) (end 125.88 94.084) (width 0.2) (layer "F.Cu") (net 10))
 (segment (start 125.88 94) (end 125.964 94) (width 0.2) (layer "F.Cu") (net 10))
 (segment (start 124.206 99.822) (end 124.206 105.664) (width 0.2) (layer "F.Cu") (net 10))
 (segment (start 125.88 94.084) (end 125.88 94) (width 0.2) (layer "F.Cu") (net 10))
 (segment (start 125.476 94.488) (end 125.476 98.552) (width 0.2) (layer "F.Cu") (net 10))
 (segment (start 124.206 105.664) (end 121.666 105.664) (width 0.2) (layer "F.Cu") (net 10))
 (segment (start 124.206 99.822) (end 125.476 98.552) (width 0.2) (layer "F.Cu") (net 10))
 (via (at 121.666 105.664) (size 0.6) (drill 0.3) (layers "F.Cu" "B.Cu") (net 10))
 (via (at 125.88 94) (size 0.6) (drill 0.3) (layers "F.Cu" "B.Cu") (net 10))
 (via (at 128.85 94.04) (size 0.6) (drill 0.3) (layers "F.Cu" "B.Cu") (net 10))
 (segment (start 113.34 104.78) (end 114.9 106.34) (width 0.2) (layer "B.Cu") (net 10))
 (segment (start 125.88 94) (end 128.81 94) (width 0.2) (layer "B.Cu") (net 10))
 (segment (start 128.81 94) (end 128.85 94.04) (width 0.2) (layer "B.Cu") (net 10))
 (segment (start 120.99 106.34) (end 121.666 105.664) (width 0.2) (layer "B.Cu") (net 10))
 (segment (start 114.9 106.34) (end 120.99 106.34) (width 0.2) (layer "B.Cu") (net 10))
 (segment (start 110.34 96.9554) (end 110.332 96.9474) (width 0.2) (layer "F.Cu") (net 9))
 (segment (start 110.34 104.78) (end 110.34 96.9554) (width 0.2) (layer "F.Cu") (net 9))
 (segment (start 110.332 96.9474) (end 110.998 96.2814) (width 0.2) (layer "F.Cu") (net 9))
 (segment (start 116.699947 100.358442) (end 117.602 101.260495) (width 0.25) (layer "F.Cu") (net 13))
 (segment (start 117.602 110.49) (end 117.094 110.998) (width 0.25) (layer "F.Cu") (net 13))
 (segment (start 116.699947 90.639547) (end 116.699947 100.358442) (width 0.25) (layer "F.Cu") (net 13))
 (segment (start 117.602 101.260495) (end 117.602 110.49) (width 0.25) (layer "F.Cu") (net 13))
 (via (at 102.2073 90.612) (size 0.8) (drill 0.4) (layers "F.Cu" "B.Cu") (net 13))
 (via (at 117.094 110.998) (size 0.8) (drill 0.4) (layers "F.Cu" "B.Cu") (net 13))
 (via (at 116.699947 90.639547) (size 0.8) (drill 0.4) (layers "F.Cu" "B.Cu") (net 13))
 (segment (start 102.234847 90.639547) (end 116.699947 90.639547) (width 0.25) (layer "B.Cu") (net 13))
 (segment (start 102.234847 90.639547) (end 102.2073 90.612) (width 0.25) (layer "B.Cu") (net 13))
 (segment (start 117.094 110.998) (end 109.4148 110.998) (width 0.25) (layer "B.Cu") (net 13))
 (segment (start 109.4148 110.998) (end 107.332 108.9152) (width 0.25) (layer "B.Cu") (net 13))
 (segment (start 107.34 107.78) (end 107.34 108.9072) (width 0.25) (layer "B.Cu") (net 13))
 (segment (start 107.34 108.9072) (end 107.332 108.9152) (width 0.2) (layer "B.Cu") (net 13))
 (segment (start 135.3058 105.203249) (end 133.074151 102.9716) (width 0.25) (layer "F.Cu") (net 14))
 (segment (start 110.34 107.78) (end 112.014 106.106) (width 0.25) (layer "F.Cu") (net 14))
 (segment (start 132.520649 102.9716) (end 132.7974 102.9716) (width 0.25) (layer "F.Cu") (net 14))
 (segment (start 131.41 101.860951) (end 132.520649 102.9716) (width 0.25) (layer "F.Cu") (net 14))
 (segment (start 131.41 99.56) (end 131.41 101.860951) (width 0.25) (layer "F.Cu") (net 14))
 (segment (start 135.3058 106.8578) (end 135.3058 105.203249) (width 0.25) (layer "F.Cu") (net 14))
 (segment (start 112.014 106.106) (end 112.014 105.49) (width 0.25) (layer "F.Cu") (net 14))
 (segment (start 112.014 105.49) (end 112.014 100.33) (width 0.25) (layer "F.Cu") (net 14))
 (segment (start 133.074151 102.9716) (end 132.7974 102.9716) (width 0.25) (layer "F.Cu") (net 14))
 (via (at 132.7974 106.7816) (size 0.8) (drill 0.4) (layers "F.Cu" "B.Cu") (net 14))
 (via (at 135.3058 106.8578) (size 0.8) (drill 0.4) (layers "F.Cu" "B.Cu") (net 14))
 (via (at 131.41 99.56) (size 0.8) (drill 0.4) (layers "F.Cu" "B.Cu") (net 14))
 (via (at 112.0114 100.3274) (size 0.8) (drill 0.4) (layers "F.Cu" "B.Cu") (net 14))
 (segment (start 131.402 99.568) (end 112.7708 99.568) (width 0.25) (layer "B.Cu") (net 14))
 (segment (start 112.7708 99.568) (end 112.0114 100.3274) (width 0.25) (layer "B.Cu") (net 14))
 (segment (start 131.41 99.56) (end 131.402 99.568) (width 0.25) (layer "B.Cu") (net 14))
 (segment (start 135.2296 106.7816) (end 135.3058 106.8578) (width 0.25) (layer "B.Cu") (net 14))
 (segment (start 132.7974 106.7816) (end 135.2296 106.7816) (width 0.25) (layer "B.Cu") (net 14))
 (segment (start 132.4102 108.0516) (end 132.3848 108.077) (width 0.25) (layer "F.Cu") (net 15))
 (segment (start 132.7974 108.0516) (end 132.4102 108.0516) (width 0.25) (layer "F.Cu") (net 15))
 (via (at 132.3848 108.077) (size 0.8) (drill 0.4) (layers "F.Cu" "B.Cu") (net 15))
 (segment (start 119.69 109.15) (end 120.06 108.78) (width 0.2) (layer "B.Cu") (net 15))
 (segment (start 126.02 107.67) (end 121.17 107.67) (width 0.25) (layer "B.Cu") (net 15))
 (segment (start 132.3848 108.077) (end 126.427 108.077) (width 0.25) (layer "B.Cu") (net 15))
 (segment (start 114.71 109.15) (end 119.69 109.15) (width 0.2) (layer "B.Cu") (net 15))
 (segment (start 126.427 108.077) (end 126.02 107.67) (width 0.25) (layer "B.Cu") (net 15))
 (segment (start 121.17 107.67) (end 120.06 108.78) (width 0.25) (layer "B.Cu") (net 15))
 (segment (start 113.34 107.78) (end 114.71 109.15) (width 0.2) (layer "B.Cu") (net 15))
 (segment (start 130.5814 103.572351) (end 132.520649 105.5116) (width 0.25) (layer "F.Cu") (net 20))
 (segment (start 130.5814 93.1926) (end 130.5814 103.572351) (width 0.25) (layer "F.Cu") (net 20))
 (segment (start 132.520649 105.5116) (end 132.7974 105.5116) (width 0.25) (layer "F.Cu") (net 20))
 (via (at 102.0826 95.184) (size 0.8) (drill 0.4) (layers "F.Cu" "B.Cu") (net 20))
 (via (at 130.5814 93.1926) (size 0.8) (drill 0.4) (layers "F.Cu" "B.Cu") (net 20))
 (segment (start 130.5814 93.1926) (end 130.5052 93.2688) (width 0.25) (layer "B.Cu") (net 20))
 (segment (start 130.5052 93.2688) (end 104.4312 93.2688) (width 0.25) (layer "B.Cu") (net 20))
 (segment (start 102.516 95.184) (end 102.0826 95.184) (width 0.25) (layer "B.Cu") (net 20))
 (segment (start 104.4312 93.2688) (end 102.516 95.184) (width 0.25) (layer "B.Cu") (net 20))
 (segment (start 125.96 102.65) (end 127.51 104.2) (width 0.2) (layer "F.Cu") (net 21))
 (segment (start 125.95 102.65) (end 125.96 102.65) (width 0.2) (layer "F.Cu") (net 21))
 (segment (start 131.4196 109.4232) (end 132.6958 109.4232) (width 0.25) (layer "F.Cu") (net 21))
 (segment (start 129.3232 109.4232) (end 131.4196 109.4232) (width 0.2) (layer "F.Cu") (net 21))
 (segment (start 127.51 104.2) (end 127.51 107.61) (width 0.2) (layer "F.Cu") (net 21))
 (segment (start 132.6958 109.4232) (end 132.7974 109.3216) (width 0.25) (layer "F.Cu") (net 21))
 (segment (start 127.51 107.61) (end 129.3232 109.4232) (width 0.2) (layer "F.Cu") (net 21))
 (via (at 137.9474 109.3216) (size 0.8) (drill 0.4) (layers "F.Cu" "B.Cu") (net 21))
 (via (at 131.4196 109.4232) (size 0.8) (drill 0.4) (layers "F.Cu" "B.Cu") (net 21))
 (segment (start 131.4196 109.4232) (end 131.5212 109.3216) (width 0.25) (layer "B.Cu") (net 21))
 (segment (start 131.5212 109.3216) (end 137.9474 109.3216) (width 0.25) (layer "B.Cu") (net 21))
 (via (at 129.032 96.266) (size 0.6) (drill 0.3) (layers "F.Cu" "B.Cu") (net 18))
 (via (at 120.142 93.98) (size 0.6) (drill 0.3) (layers "F.Cu" "B.Cu") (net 18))
 (segment (start 128.016 95.25) (end 129.032 96.266) (width 0.2) (layer "B.Cu") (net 18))
 (segment (start 120.142 93.98) (end 121.412 95.25) (width 0.2) (layer "B.Cu") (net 18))
 (segment (start 121.412 95.25) (end 128.016 95.25) (width 0.2) (layer "B.Cu") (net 18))
 (via (at 111.252 93.98) (size 0.6) (drill 0.3) (layers "F.Cu" "B.Cu") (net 17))
 (via (at 120.142 96.266) (size 0.6) (drill 0.3) (layers "F.Cu" "B.Cu") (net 17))
 (segment (start 119.126 95.25) (end 120.142 96.266) (width 0.2) (layer "B.Cu") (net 17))
 (segment (start 112.522 95.25) (end 119.126 95.25) (width 0.2) (layer "B.Cu") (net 17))
 (segment (start 111.252 93.98) (end 112.522 95.25) (width 0.2) (layer "B.Cu") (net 17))
 (via (at 120.03 88.71) (size 0.6) (drill 0.3) (layers "F.Cu" "B.Cu") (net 19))
 (via (at 100.4 94.28) (size 0.6) (drill 0.3) (layers "F.Cu" "B.Cu") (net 19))
 (segment (start 120.09 88.71) (end 120.04 88.76) (width 0.2) (layer "B.Cu") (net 19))
 (segment (start 120.03 88.71) (end 120.09 88.71) (width 0.2) (layer "B.Cu") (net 19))
 (segment (start 120.03 88.77) (end 120.03 88.71) (width 0.2) (layer "B.Cu") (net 19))
 (segment (start 100.4 94.28) (end 102.53 94.28) (width 0.2) (layer "B.Cu") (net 19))
 (segment (start 102.53 94.28) (end 104.59 92.22) (width 0.2) (layer "B.Cu") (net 19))
 (segment (start 119.9 88.9) (end 120.03 88.77) (width 0.2) (layer "B.Cu") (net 19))
 (segment (start 104.59 92.22) (end 118.3 92.22) (width 0.2) (layer "B.Cu") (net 19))
 (segment (start 118.3 92.22) (end 119.9 90.62) (width 0.2) (layer "B.Cu") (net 19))
 (segment (start 119.9 90.62) (end 119.9 88.9) (width 0.2) (layer "B.Cu") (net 19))
 (segment (start 126.9 100.775) (end 126.9 90.77) (width 0.2) (layer "F.Cu") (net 23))
 (segment (start 128.9304 88.7396) (end 128.9304 88.6714) (width 0.2) (layer "F.Cu") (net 23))
 (segment (start 126.9 90.77) (end 128.9304 88.7396) (width 0.2) (layer "F.Cu") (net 23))
 (segment (start 100.3323 89.662) (end 100.41 89.61) (width 0.2) (layer "F.Cu") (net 24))
 (via (at 110.55 88.72) (size 0.6) (drill 0.3) (layers "F.Cu" "B.Cu") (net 24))
 (via (at 100.41 89.61) (size 0.6) (drill 0.3) (layers "F.Cu" "B.Cu") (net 24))
 (segment (start 100.41 89.61) (end 109.66 89.61) (width 0.2) (layer "B.Cu") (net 24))
 (segment (start 109.66 89.61) (end 110.55 88.72) (width 0.2) (layer "B.Cu") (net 24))
 (via (at 137.414 96.266) (size 0.6) (drill 0.3) (layers "F.Cu" "B.Cu") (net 6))
 (segment (start 131.098 106.9) (end 131.953 106.045) (width 0.2) (layer "B.Cu") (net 6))
 (segment (start 136.017 106.045) (end 136.652 105.41) (width 0.2) (layer "B.Cu") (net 6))
 (segment (start 119.34 107.78) (end 120.22 106.9) (width 0.2) (layer "B.Cu") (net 6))
 (segment (start 120.22 106.9) (end 131.098 106.9) (width 0.2) (layer "B.Cu") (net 6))
 (segment (start 131.953 106.045) (end 136.017 106.045) (width 0.2) (layer "B.Cu") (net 6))
 (segment (start 136.652 97.028) (end 137.414 96.266) (width 0.2) (layer "B.Cu") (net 6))
 (segment (start 136.652 105.41) (end 136.652 97.028) (width 0.2) (layer "B.Cu") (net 6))
 (segment (start 116.34 113.25) (end 116.34 108.9072) (width 0.2) (layer "F.Cu") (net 3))
 (segment (start 139.33 97.6) (end 136.31 100.62) (width 0.2) (layer "F.Cu") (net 3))
 (segment (start 135.2126 91.55) (end 137.89 91.55) (width 0.2) (layer "F.Cu") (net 3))
 (segment (start 136.31 100.62) (end 136.31 111.95) (width 0.2) (layer "F.Cu") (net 3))
 (segment (start 139.33 92.99) (end 139.33 97.6) (width 0.2) (layer "F.Cu") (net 3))
 (segment (start 136.31 111.95) (end 133.36 114.9) (width 0.2) (layer "F.Cu") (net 3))
 (segment (start 116.34 108.9072) (end 116.34 107.78) (width 0.2) (layer "F.Cu") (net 3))
 (segment (start 137.89 91.55) (end 139.33 92.99) (width 0.2) (layer "F.Cu") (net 3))
 (segment (start 116.34 108.9072) (end 116.332 108.9152) (width 0.2) (layer "F.Cu") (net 3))
 (segment (start 117.99 114.9) (end 116.34 113.25) (width 0.2) (layer "F.Cu") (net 3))
 (segment (start 133.36 114.9) (end 117.99 114.9) (width 0.2) (layer "F.Cu") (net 3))
 (segment (start 132.2324 88.5698) (end 135.2126 91.55) (width 0.2) (layer "F.Cu") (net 3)))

